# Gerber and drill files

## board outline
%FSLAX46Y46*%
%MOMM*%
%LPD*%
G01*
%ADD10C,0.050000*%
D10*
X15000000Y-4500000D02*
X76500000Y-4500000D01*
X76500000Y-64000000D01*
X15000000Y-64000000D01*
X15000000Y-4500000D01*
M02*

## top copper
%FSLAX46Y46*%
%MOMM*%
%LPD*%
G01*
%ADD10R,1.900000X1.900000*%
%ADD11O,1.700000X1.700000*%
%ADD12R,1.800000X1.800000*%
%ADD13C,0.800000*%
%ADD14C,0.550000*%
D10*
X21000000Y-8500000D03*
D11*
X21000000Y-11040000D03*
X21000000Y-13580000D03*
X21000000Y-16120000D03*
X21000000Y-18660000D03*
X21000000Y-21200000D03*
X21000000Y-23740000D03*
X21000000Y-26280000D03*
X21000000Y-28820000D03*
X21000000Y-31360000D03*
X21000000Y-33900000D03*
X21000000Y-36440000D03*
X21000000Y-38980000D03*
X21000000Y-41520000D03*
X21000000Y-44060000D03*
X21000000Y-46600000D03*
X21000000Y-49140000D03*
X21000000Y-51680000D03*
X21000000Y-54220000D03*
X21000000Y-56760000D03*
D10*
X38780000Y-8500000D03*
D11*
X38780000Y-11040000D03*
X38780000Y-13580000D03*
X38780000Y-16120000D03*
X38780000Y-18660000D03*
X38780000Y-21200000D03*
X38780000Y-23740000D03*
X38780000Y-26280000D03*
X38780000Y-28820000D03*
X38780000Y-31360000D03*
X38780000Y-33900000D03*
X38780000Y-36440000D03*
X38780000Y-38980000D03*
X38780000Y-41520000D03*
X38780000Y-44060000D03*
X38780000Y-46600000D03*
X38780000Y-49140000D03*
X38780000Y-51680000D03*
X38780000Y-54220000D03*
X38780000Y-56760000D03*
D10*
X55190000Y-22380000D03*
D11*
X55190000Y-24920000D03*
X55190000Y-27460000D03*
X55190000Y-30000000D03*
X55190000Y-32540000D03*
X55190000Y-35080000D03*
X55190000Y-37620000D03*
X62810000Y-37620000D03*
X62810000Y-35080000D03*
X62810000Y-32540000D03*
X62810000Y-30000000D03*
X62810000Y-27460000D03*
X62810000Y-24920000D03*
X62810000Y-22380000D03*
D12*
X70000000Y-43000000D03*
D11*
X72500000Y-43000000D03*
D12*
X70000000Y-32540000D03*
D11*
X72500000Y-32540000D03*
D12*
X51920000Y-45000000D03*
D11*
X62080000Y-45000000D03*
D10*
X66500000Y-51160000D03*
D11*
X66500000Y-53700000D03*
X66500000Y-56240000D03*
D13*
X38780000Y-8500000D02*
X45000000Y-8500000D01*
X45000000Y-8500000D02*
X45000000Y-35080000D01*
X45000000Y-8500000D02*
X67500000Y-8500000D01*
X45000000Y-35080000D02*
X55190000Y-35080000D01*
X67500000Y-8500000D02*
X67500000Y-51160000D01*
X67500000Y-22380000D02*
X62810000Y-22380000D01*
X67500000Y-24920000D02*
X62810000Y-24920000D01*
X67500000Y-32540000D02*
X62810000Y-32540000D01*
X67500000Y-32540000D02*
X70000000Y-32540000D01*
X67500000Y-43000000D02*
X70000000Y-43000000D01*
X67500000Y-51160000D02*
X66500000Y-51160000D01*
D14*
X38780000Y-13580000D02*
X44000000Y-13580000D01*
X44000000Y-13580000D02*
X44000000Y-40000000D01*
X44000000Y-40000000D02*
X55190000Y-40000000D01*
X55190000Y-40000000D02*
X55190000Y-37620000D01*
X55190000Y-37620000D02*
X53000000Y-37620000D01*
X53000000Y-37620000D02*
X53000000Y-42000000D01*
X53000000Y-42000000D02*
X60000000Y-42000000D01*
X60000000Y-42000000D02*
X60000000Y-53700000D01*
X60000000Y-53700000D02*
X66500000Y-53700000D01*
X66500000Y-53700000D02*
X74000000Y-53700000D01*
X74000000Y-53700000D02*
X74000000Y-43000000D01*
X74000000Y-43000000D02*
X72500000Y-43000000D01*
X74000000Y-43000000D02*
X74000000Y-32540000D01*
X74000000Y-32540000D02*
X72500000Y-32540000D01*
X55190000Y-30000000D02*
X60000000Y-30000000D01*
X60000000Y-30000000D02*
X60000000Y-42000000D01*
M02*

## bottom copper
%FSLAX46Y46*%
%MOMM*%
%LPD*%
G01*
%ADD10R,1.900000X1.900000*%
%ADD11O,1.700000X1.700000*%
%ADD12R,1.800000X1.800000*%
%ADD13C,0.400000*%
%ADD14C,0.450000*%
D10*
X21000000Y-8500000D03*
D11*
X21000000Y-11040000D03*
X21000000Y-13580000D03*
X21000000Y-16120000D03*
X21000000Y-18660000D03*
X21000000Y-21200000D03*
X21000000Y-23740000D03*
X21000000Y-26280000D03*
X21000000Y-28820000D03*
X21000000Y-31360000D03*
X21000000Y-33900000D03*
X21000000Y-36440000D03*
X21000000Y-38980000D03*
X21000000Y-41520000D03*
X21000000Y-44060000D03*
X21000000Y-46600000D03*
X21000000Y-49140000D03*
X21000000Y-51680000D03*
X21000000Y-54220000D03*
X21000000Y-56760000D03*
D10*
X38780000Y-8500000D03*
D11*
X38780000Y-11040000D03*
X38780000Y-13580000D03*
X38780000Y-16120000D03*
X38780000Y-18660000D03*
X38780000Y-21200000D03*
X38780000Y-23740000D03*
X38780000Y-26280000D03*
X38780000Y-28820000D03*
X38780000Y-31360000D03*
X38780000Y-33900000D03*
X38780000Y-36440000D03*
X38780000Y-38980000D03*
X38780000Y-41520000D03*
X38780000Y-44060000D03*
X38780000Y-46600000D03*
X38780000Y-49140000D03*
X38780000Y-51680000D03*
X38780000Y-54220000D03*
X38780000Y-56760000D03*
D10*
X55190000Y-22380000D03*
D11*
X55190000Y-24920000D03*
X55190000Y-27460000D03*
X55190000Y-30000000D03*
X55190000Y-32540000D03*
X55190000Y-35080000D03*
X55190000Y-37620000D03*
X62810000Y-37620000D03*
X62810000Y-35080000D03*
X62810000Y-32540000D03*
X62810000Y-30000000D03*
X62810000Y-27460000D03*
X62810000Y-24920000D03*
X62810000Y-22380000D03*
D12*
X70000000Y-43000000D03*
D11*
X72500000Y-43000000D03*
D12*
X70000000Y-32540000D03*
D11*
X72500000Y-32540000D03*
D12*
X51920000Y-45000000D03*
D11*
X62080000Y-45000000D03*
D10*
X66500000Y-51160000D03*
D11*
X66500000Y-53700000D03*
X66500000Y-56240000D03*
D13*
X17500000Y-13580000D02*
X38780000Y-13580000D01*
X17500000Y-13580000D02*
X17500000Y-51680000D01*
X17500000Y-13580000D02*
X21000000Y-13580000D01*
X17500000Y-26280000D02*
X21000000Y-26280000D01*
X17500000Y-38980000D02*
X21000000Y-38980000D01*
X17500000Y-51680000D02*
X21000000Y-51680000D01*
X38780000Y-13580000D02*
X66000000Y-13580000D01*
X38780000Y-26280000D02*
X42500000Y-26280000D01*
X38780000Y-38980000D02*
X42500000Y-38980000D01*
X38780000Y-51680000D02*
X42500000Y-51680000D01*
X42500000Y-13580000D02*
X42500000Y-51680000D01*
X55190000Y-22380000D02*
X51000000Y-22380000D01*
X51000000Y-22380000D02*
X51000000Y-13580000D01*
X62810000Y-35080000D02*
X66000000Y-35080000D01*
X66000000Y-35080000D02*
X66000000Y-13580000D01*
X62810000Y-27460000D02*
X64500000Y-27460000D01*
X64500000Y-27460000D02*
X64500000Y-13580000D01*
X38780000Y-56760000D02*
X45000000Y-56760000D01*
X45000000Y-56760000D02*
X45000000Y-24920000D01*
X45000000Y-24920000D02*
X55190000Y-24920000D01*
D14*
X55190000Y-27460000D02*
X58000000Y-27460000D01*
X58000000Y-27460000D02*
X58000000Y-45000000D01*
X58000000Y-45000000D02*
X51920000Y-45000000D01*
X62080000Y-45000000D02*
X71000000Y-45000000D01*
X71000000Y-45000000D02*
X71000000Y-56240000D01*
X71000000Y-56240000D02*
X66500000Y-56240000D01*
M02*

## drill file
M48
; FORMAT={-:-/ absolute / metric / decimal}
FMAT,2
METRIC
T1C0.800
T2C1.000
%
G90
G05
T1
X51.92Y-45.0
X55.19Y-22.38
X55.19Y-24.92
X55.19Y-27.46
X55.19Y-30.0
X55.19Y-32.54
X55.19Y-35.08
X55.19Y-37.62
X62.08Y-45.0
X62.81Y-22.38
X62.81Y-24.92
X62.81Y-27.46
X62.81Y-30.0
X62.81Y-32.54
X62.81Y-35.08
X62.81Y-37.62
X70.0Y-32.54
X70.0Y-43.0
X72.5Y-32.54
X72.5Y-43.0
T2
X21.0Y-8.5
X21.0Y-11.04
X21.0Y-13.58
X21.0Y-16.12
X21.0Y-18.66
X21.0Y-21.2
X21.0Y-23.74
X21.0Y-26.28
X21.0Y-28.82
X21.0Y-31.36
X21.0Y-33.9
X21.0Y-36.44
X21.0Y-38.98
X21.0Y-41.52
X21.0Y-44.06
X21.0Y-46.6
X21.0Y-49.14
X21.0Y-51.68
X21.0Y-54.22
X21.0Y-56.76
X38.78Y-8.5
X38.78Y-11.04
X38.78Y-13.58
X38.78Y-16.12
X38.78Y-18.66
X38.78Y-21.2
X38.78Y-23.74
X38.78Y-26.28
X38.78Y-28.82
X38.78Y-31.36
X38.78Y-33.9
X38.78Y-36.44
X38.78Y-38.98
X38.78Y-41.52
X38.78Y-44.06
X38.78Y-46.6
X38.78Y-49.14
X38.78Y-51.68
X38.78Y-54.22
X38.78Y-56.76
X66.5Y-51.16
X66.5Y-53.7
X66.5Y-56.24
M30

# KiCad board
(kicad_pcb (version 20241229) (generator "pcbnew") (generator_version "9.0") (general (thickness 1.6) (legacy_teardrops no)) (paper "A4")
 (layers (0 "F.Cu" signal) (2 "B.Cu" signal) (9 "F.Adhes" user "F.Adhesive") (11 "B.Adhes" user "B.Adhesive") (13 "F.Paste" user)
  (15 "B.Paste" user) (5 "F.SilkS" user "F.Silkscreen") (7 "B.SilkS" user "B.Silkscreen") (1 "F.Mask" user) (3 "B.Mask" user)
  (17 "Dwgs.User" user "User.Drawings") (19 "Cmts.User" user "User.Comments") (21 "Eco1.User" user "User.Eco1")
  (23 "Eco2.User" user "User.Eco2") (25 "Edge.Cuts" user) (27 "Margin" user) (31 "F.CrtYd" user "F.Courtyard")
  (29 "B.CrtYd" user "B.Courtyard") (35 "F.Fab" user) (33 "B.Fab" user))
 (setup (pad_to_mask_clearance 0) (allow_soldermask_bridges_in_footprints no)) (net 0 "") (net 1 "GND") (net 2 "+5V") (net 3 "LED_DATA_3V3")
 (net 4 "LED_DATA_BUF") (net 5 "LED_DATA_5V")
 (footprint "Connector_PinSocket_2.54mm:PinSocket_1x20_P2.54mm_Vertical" (layer "F.Cu") (at 21 8.5)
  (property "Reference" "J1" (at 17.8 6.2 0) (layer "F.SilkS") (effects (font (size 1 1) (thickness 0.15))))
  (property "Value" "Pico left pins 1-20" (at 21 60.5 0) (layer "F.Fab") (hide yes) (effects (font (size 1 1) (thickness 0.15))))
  (pad "1" thru_hole rect (at 0 0) (size 1.9 1.9) (drill 1) (layers "*.Cu" "*.Mask") (remove_unused_layers no) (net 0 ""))
  (pad "2" thru_hole oval (at 0 2.54) (size 1.7 1.7) (drill 1) (layers "*.Cu" "*.Mask") (remove_unused_layers no) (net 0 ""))
  (pad "3" thru_hole oval (at 0 5.08) (size 1.7 1.7) (drill 1) (layers "*.Cu" "*.Mask") (remove_unused_layers no) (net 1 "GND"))
  (pad "4" thru_hole oval (at 0 7.62) (size 1.7 1.7) (drill 1) (layers "*.Cu" "*.Mask") (remove_unused_layers no) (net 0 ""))
  (pad "5" thru_hole oval (at 0 10.16) (size 1.7 1.7) (drill 1) (layers "*.Cu" "*.Mask") (remove_unused_layers no) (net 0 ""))
  (pad "6" thru_hole oval (at 0 12.7) (size 1.7 1.7) (drill 1) (layers "*.Cu" "*.Mask") (remove_unused_layers no) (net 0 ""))
  (pad "7" thru_hole oval (at 0 15.24) (size 1.7 1.7) (drill 1) (layers "*.Cu" "*.Mask") (remove_unused_layers no) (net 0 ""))
  (pad "8" thru_hole oval (at 0 17.78) (size 1.7 1.7) (drill 1) (layers "*.Cu" "*.Mask") (remove_unused_layers no) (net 1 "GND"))
  (pad "9" thru_hole oval (at 0 20.32) (size 1.7 1.7) (drill 1) (layers "*.Cu" "*.Mask") (remove_unused_layers no) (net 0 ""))
  (pad "10" thru_hole oval (at 0 22.86) (size 1.7 1.7) (drill 1) (layers "*.Cu" "*.Mask") (remove_unused_layers no) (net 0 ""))
  (pad "11" thru_hole oval (at 0 25.4) (size 1.7 1.7) (drill 1) (layers "*.Cu" "*.Mask") (remove_unused_layers no) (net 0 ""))
  (pad "12" thru_hole oval (at 0 27.94) (size 1.7 1.7) (drill 1) (layers "*.Cu" "*.Mask") (remove_unused_layers no) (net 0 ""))
  (pad "13" thru_hole oval (at 0 30.48) (size 1.7 1.7) (drill 1) (layers "*.Cu" "*.Mask") (remove_unused_layers no) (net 1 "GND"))
  (pad "14" thru_hole oval (at 0 33.02) (size 1.7 1.7) (drill 1) (layers "*.Cu" "*.Mask") (remove_unused_layers no) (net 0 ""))
  (pad "15" thru_hole oval (at 0 35.56) (size 1.7 1.7) (drill 1) (layers "*.Cu" "*.Mask") (remove_unused_layers no) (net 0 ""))
  (pad "16" thru_hole oval (at 0 38.1) (size 1.7 1.7) (drill 1) (layers "*.Cu" "*.Mask") (remove_unused_layers no) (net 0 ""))
  (pad "17" thru_hole oval (at 0 40.64) (size 1.7 1.7) (drill 1) (layers "*.Cu" "*.Mask") (remove_unused_layers no) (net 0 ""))
  (pad "18" thru_hole oval (at 0 43.18) (size 1.7 1.7) (drill 1) (layers "*.Cu" "*.Mask") (remove_unused_layers no) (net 1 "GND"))
  (pad "19" thru_hole oval (at 0 45.72) (size 1.7 1.7) (drill 1) (layers "*.Cu" "*.Mask") (remove_unused_layers no) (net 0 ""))
  (pad "20" thru_hole oval (at 0 48.26) (size 1.7 1.7) (drill 1) (layers "*.Cu" "*.Mask") (remove_unused_layers no) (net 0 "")))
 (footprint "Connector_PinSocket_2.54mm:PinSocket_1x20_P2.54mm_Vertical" (layer "F.Cu") (at 38.78 8.5)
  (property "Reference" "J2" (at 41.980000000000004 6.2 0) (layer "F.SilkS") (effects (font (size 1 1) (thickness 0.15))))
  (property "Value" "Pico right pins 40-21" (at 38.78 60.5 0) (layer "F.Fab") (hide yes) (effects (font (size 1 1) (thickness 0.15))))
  (pad "1" thru_hole rect (at 0 0) (size 1.9 1.9) (drill 1) (layers "*.Cu" "*.Mask") (remove_unused_layers no) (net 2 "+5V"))
  (pad "2" thru_hole oval (at 0 2.54) (size 1.7 1.7) (drill 1) (layers "*.Cu" "*.Mask") (remove_unused_layers no) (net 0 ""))
  (pad "3" thru_hole oval (at 0 5.08) (size 1.7 1.7) (drill 1) (layers "*.Cu" "*.Mask") (remove_unused_layers no) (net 1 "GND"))
  (pad "4" thru_hole oval (at 0 7.62) (size 1.7 1.7) (drill 1) (layers "*.Cu" "*.Mask") (remove_unused_layers no) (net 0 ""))
  (pad "5" thru_hole oval (at 0 10.16) (size 1.7 1.7) (drill 1) (layers "*.Cu" "*.Mask") (remove_unused_layers no) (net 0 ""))
  (pad "6" thru_hole oval (at 0 12.7) (size 1.7 1.7) (drill 1) (layers "*.Cu" "*.Mask") (remove_unused_layers no) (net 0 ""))
  (pad "7" thru_hole oval (at 0 15.24) (size 1.7 1.7) (drill 1) (layers "*.Cu" "*.Mask") (remove_unused_layers no) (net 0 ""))
  (pad "8" thru_hole oval (at 0 17.78) (size 1.7 1.7) (drill 1) (layers "*.Cu" "*.Mask") (remove_unused_layers no) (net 1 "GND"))
  (pad "9" thru_hole oval (at 0 20.32) (size 1.7 1.7) (drill 1) (layers "*.Cu" "*.Mask") (remove_unused_layers no) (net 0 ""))
  (pad "10" thru_hole oval (at 0 22.86) (size 1.7 1.7) (drill 1) (layers "*.Cu" "*.Mask") (remove_unused_layers no) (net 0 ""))
  (pad "11" thru_hole oval (at 0 25.4) (size 1.7 1.7) (drill 1) (layers "*.Cu" "*.Mask") (remove_unused_layers no) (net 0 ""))
  (pad "12" thru_hole oval (at 0 27.94) (size 1.7 1.7) (drill 1) (layers "*.Cu" "*.Mask") (remove_unused_layers no) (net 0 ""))
  (pad "13" thru_hole oval (at 0 30.48) (size 1.7 1.7) (drill 1) (layers "*.Cu" "*.Mask") (remove_unused_layers no) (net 1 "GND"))
  (pad "14" thru_hole oval (at 0 33.02) (size 1.7 1.7) (drill 1) (layers "*.Cu" "*.Mask") (remove_unused_layers no) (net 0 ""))
  (pad "15" thru_hole oval (at 0 35.56) (size 1.7 1.7) (drill 1) (layers "*.Cu" "*.Mask") (remove_unused_layers no) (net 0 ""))
  (pad "16" thru_hole oval (at 0 38.1) (size 1.7 1.7) (drill 1) (layers "*.Cu" "*.Mask") (remove_unused_layers no) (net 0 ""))
  (pad "17" thru_hole oval (at 0 40.64) (size 1.7 1.7) (drill 1) (layers "*.Cu" "*.Mask") (remove_unused_layers no) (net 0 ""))
  (pad "18" thru_hole oval (at 0 43.18) (size 1.7 1.7) (drill 1) (layers "*.Cu" "*.Mask") (remove_unused_layers no) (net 1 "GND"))
  (pad "19" thru_hole oval (at 0 45.72) (size 1.7 1.7) (drill 1) (layers "*.Cu" "*.Mask") (remove_unused_layers no) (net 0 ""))
  (pad "20" thru_hole oval (at 0 48.26) (size 1.7 1.7) (drill 1) (layers "*.Cu" "*.Mask") (remove_unused_layers no) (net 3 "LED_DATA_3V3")))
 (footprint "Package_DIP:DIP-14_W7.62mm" (layer "F.Cu") (at 55.19 22.38)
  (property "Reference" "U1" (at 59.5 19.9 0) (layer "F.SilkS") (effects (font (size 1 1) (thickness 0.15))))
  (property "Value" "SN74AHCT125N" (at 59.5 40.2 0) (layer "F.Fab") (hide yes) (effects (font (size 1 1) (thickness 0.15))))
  (pad "1" thru_hole rect (at 0 0) (size 1.9 1.9) (drill 0.8) (layers "*.Cu" "*.Mask") (remove_unused_layers no) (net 1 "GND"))
  (pad "2" thru_hole oval (at 0 2.54) (size 1.7 1.7) (drill 0.8) (layers "*.Cu" "*.Mask") (remove_unused_layers no) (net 3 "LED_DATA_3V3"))
  (pad "3" thru_hole oval (at 0 5.08) (size 1.7 1.7) (drill 0.8) (layers "*.Cu" "*.Mask") (remove_unused_layers no) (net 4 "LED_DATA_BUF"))
  (pad "4" thru_hole oval (at 0 7.62) (size 1.7 1.7) (drill 0.8) (layers "*.Cu" "*.Mask") (remove_unused_layers no) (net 1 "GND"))
  (pad "5" thru_hole oval (at 0 10.16) (size 1.7 1.7) (drill 0.8) (layers "*.Cu" "*.Mask") (remove_unused_layers no) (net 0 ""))
  (pad "6" thru_hole oval (at 0 12.7) (size 1.7 1.7) (drill 0.8) (layers "*.Cu" "*.Mask") (remove_unused_layers no) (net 2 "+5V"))
  (pad "7" thru_hole oval (at 0 15.24) (size 1.7 1.7) (drill 0.8) (layers "*.Cu" "*.Mask") (remove_unused_layers no) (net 1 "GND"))
  (pad "8" thru_hole oval (at 7.62 15.24) (size 1.7 1.7) (drill 0.8) (layers "*.Cu" "*.Mask") (remove_unused_layers no) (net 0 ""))
  (pad "9" thru_hole oval (at 7.62 12.7) (size 1.7 1.7) (drill 0.8) (layers "*.Cu" "*.Mask") (remove_unused_layers no) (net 1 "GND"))
  (pad "10" thru_hole oval (at 7.62 10.16) (size 1.7 1.7) (drill 0.8) (layers "*.Cu" "*.Mask") (remove_unused_layers no) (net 2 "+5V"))
  (pad "11" thru_hole oval (at 7.62 7.62) (size 1.7 1.7) (drill 0.8) (layers "*.Cu" "*.Mask") (remove_unused_layers no) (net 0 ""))
  (pad "12" thru_hole oval (at 7.62 5.08) (size 1.7 1.7) (drill 0.8) (layers "*.Cu" "*.Mask") (remove_unused_layers no) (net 1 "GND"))
  (pad "13" thru_hole oval (at 7.62 2.54) (size 1.7 1.7) (drill 0.8) (layers "*.Cu" "*.Mask") (remove_unused_layers no) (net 2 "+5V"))
  (pad "14" thru_hole oval (at 7.62 0) (size 1.7 1.7) (drill 0.8) (layers "*.Cu" "*.Mask") (remove_unused_layers no) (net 2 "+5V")))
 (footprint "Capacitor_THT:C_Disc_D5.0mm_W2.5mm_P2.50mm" (layer "F.Cu") (at 70 43)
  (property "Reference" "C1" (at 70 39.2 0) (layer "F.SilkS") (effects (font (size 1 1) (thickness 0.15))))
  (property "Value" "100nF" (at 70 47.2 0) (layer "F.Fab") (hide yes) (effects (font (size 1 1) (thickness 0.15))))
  (pad "1" thru_hole rect (at 0 0) (size 1.8 1.8) (drill 0.8) (layers "*.Cu" "*.Mask") (remove_unused_layers no) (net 2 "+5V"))
  (pad "2" thru_hole oval (at 2.5 0) (size 1.7 1.7) (drill 0.8) (layers "*.Cu" "*.Mask") (remove_unused_layers no) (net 1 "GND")))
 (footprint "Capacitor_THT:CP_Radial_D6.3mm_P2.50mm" (layer "F.Cu") (at 70 32.54)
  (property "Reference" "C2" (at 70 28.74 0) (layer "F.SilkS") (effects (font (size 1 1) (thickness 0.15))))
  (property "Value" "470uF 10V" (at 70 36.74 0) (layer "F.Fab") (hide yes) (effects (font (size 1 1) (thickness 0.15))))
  (pad "1" thru_hole rect (at 0 0) (size 1.8 1.8) (drill 0.8) (layers "*.Cu" "*.Mask") (remove_unused_layers no) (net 2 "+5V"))
  (pad "2" thru_hole oval (at 2.5 0) (size 1.7 1.7) (drill 0.8) (layers "*.Cu" "*.Mask") (remove_unused_layers no) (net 1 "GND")))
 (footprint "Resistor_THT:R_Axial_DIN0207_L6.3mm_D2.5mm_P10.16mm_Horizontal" (layer "F.Cu") (at 57 45)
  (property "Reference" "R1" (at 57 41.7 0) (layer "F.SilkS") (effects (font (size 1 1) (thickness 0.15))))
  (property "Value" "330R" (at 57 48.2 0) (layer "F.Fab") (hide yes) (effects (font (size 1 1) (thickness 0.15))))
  (pad "1" thru_hole rect (at -5.08 0) (size 1.8 1.8) (drill 0.8) (layers "*.Cu" "*.Mask") (remove_unused_layers no) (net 4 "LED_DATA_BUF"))
  (pad "2" thru_hole oval (at 5.08 0) (size 1.7 1.7) (drill 0.8) (layers "*.Cu" "*.Mask") (remove_unused_layers no) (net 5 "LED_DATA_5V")))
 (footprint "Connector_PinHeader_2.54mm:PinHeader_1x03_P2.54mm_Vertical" (layer "F.Cu") (at 66.5 51.16)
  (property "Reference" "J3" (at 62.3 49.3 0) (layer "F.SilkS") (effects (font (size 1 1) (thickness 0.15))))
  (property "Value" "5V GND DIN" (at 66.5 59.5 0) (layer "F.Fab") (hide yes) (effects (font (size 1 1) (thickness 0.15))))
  (pad "1" thru_hole rect (at 0 0) (size 1.9 1.9) (drill 1) (layers "*.Cu" "*.Mask") (remove_unused_layers no) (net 2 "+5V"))
  (pad "2" thru_hole oval (at 0 2.54) (size 1.7 1.7) (drill 1) (layers "*.Cu" "*.Mask") (remove_unused_layers no) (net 1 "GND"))
  (pad "3" thru_hole oval (at 0 5.08) (size 1.7 1.7) (drill 1) (layers "*.Cu" "*.Mask") (remove_unused_layers no) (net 5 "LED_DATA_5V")))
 (gr_rect (start 15 4.5) (end 76.5 64) (stroke (width 0.05) (type solid)) (fill none) (layer "Edge.Cuts"))
 (segment (start 38.78 8.5) (end 45 8.5) (width 0.8) (layer "F.Cu") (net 2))
 (segment (start 45 8.5) (end 45 35.08) (width 0.8) (layer "F.Cu") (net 2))
 (segment (start 45 8.5) (end 67.5 8.5) (width 0.8) (layer "F.Cu") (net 2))
 (segment (start 45 35.08) (end 55.19 35.08) (width 0.8) (layer "F.Cu") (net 2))
 (segment (start 67.5 8.5) (end 67.5 51.16) (width 0.8) (layer "F.Cu") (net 2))
 (segment (start 67.5 22.38) (end 62.81 22.38) (width 0.8) (layer "F.Cu") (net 2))
 (segment (start 67.5 24.92) (end 62.81 24.92) (width 0.8) (layer "F.Cu") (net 2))
 (segment (start 67.5 32.54) (end 62.81 32.54) (width 0.8) (layer "F.Cu") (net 2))
 (segment (start 67.5 32.54) (end 70 32.54) (width 0.8) (layer "F.Cu") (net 2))
 (segment (start 67.5 43) (end 70 43) (width 0.8) (layer "F.Cu") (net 2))
 (segment (start 67.5 51.16) (end 66.5 51.16) (width 0.8) (layer "F.Cu") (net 2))
 (segment (start 38.78 13.58) (end 44 13.58) (width 0.55) (layer "F.Cu") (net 1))
 (segment (start 44 13.58) (end 44 40) (width 0.55) (layer "F.Cu") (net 1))
 (segment (start 44 40) (end 55.19 40) (width 0.55) (layer "F.Cu") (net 1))
 (segment (start 55.19 40) (end 55.19 37.62) (width 0.55) (layer "F.Cu") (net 1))
 (segment (start 55.19 37.62) (end 53 37.62) (width 0.55) (layer "F.Cu") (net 1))
 (segment (start 53 37.62) (end 53 42) (width 0.55) (layer "F.Cu") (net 1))
 (segment (start 53 42) (end 60 42) (width 0.55) (layer "F.Cu") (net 1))
 (segment (start 60 42) (end 60 53.7) (width 0.55) (layer "F.Cu") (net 1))
 (segment (start 60 53.7) (end 66.5 53.7) (width 0.55) (layer "F.Cu") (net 1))
 (segment (start 66.5 53.7) (end 74 53.7) (width 0.55) (layer "F.Cu") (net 1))
 (segment (start 74 53.7) (end 74 43) (width 0.55) (layer "F.Cu") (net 1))
 (segment (start 74 43) (end 72.5 43) (width 0.55) (layer "F.Cu") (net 1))
 (segment (start 74 43) (end 74 32.54) (width 0.55) (layer "F.Cu") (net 1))
 (segment (start 74 32.54) (end 72.5 32.54) (width 0.55) (layer "F.Cu") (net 1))
 (segment (start 17.5 13.58) (end 38.78 13.58) (width 0.4) (layer "B.Cu") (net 1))
 (segment (start 17.5 13.58) (end 17.5 51.68) (width 0.4) (layer "B.Cu") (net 1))
 (segment (start 17.5 13.58) (end 21 13.58) (width 0.4) (layer "B.Cu") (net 1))
 (segment (start 17.5 26.28) (end 21 26.28) (width 0.4) (layer "B.Cu") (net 1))
 (segment (start 17.5 38.98) (end 21 38.98) (width 0.4) (layer "B.Cu") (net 1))
 (segment (start 17.5 51.68) (end 21 51.68) (width 0.4) (layer "B.Cu") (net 1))
 (segment (start 38.78 13.58) (end 66 13.58) (width 0.4) (layer "B.Cu") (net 1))
 (segment (start 38.78 26.28) (end 42.5 26.28) (width 0.4) (layer "B.Cu") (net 1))
 (segment (start 38.78 38.98) (end 42.5 38.98) (width 0.4) (layer "B.Cu") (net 1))
 (segment (start 38.78 51.68) (end 42.5 51.68) (width 0.4) (layer "B.Cu") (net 1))
 (segment (start 42.5 13.58) (end 42.5 51.68) (width 0.4) (layer "B.Cu") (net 1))
 (segment (start 55.19 22.38) (end 51 22.38) (width 0.4) (layer "B.Cu") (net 1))
 (segment (start 51 22.38) (end 51 13.58) (width 0.4) (layer "B.Cu") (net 1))
 (segment (start 55.19 30) (end 60 30) (width 0.55) (layer "F.Cu") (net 1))
 (segment (start 60 30) (end 60 42) (width 0.55) (layer "F.Cu") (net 1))
 (segment (start 62.81 35.08) (end 66 35.08) (width 0.4) (layer "B.Cu") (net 1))
 (segment (start 66 35.08) (end 66 13.58) (width 0.4) (layer "B.Cu") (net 1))
 (segment (start 62.81 27.46) (end 64.5 27.46) (width 0.4) (layer "B.Cu") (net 1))
 (segment (start 64.5 27.46) (end 64.5 13.58) (width 0.4) (layer "B.Cu") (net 1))
 (segment (start 38.78 56.76) (end 45 56.76) (width 0.4) (layer "B.Cu") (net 3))
 (segment (start 45 56.76) (end 45 24.92) (width 0.4) (layer "B.Cu") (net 3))
 (segment (start 45 24.92) (end 55.19 24.92) (width 0.4) (layer "B.Cu") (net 3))
 (segment (start 55.19 27.46) (end 58 27.46) (width 0.45) (layer "B.Cu") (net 4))
 (segment (start 58 27.46) (end 58 45) (width 0.45) (layer "B.Cu") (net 4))
 (segment (start 58 45) (end 51.92 45) (width 0.45) (layer "B.Cu") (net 4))
 (segment (start 62.08 45) (end 71 45) (width 0.45) (layer "B.Cu") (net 5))
 (segment (start 71 45) (end 71 56.24) (width 0.45) (layer "B.Cu") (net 5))
 (segment (start 71 56.24) (end 66.5 56.24) (width 0.45) (layer "B.Cu") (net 5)))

